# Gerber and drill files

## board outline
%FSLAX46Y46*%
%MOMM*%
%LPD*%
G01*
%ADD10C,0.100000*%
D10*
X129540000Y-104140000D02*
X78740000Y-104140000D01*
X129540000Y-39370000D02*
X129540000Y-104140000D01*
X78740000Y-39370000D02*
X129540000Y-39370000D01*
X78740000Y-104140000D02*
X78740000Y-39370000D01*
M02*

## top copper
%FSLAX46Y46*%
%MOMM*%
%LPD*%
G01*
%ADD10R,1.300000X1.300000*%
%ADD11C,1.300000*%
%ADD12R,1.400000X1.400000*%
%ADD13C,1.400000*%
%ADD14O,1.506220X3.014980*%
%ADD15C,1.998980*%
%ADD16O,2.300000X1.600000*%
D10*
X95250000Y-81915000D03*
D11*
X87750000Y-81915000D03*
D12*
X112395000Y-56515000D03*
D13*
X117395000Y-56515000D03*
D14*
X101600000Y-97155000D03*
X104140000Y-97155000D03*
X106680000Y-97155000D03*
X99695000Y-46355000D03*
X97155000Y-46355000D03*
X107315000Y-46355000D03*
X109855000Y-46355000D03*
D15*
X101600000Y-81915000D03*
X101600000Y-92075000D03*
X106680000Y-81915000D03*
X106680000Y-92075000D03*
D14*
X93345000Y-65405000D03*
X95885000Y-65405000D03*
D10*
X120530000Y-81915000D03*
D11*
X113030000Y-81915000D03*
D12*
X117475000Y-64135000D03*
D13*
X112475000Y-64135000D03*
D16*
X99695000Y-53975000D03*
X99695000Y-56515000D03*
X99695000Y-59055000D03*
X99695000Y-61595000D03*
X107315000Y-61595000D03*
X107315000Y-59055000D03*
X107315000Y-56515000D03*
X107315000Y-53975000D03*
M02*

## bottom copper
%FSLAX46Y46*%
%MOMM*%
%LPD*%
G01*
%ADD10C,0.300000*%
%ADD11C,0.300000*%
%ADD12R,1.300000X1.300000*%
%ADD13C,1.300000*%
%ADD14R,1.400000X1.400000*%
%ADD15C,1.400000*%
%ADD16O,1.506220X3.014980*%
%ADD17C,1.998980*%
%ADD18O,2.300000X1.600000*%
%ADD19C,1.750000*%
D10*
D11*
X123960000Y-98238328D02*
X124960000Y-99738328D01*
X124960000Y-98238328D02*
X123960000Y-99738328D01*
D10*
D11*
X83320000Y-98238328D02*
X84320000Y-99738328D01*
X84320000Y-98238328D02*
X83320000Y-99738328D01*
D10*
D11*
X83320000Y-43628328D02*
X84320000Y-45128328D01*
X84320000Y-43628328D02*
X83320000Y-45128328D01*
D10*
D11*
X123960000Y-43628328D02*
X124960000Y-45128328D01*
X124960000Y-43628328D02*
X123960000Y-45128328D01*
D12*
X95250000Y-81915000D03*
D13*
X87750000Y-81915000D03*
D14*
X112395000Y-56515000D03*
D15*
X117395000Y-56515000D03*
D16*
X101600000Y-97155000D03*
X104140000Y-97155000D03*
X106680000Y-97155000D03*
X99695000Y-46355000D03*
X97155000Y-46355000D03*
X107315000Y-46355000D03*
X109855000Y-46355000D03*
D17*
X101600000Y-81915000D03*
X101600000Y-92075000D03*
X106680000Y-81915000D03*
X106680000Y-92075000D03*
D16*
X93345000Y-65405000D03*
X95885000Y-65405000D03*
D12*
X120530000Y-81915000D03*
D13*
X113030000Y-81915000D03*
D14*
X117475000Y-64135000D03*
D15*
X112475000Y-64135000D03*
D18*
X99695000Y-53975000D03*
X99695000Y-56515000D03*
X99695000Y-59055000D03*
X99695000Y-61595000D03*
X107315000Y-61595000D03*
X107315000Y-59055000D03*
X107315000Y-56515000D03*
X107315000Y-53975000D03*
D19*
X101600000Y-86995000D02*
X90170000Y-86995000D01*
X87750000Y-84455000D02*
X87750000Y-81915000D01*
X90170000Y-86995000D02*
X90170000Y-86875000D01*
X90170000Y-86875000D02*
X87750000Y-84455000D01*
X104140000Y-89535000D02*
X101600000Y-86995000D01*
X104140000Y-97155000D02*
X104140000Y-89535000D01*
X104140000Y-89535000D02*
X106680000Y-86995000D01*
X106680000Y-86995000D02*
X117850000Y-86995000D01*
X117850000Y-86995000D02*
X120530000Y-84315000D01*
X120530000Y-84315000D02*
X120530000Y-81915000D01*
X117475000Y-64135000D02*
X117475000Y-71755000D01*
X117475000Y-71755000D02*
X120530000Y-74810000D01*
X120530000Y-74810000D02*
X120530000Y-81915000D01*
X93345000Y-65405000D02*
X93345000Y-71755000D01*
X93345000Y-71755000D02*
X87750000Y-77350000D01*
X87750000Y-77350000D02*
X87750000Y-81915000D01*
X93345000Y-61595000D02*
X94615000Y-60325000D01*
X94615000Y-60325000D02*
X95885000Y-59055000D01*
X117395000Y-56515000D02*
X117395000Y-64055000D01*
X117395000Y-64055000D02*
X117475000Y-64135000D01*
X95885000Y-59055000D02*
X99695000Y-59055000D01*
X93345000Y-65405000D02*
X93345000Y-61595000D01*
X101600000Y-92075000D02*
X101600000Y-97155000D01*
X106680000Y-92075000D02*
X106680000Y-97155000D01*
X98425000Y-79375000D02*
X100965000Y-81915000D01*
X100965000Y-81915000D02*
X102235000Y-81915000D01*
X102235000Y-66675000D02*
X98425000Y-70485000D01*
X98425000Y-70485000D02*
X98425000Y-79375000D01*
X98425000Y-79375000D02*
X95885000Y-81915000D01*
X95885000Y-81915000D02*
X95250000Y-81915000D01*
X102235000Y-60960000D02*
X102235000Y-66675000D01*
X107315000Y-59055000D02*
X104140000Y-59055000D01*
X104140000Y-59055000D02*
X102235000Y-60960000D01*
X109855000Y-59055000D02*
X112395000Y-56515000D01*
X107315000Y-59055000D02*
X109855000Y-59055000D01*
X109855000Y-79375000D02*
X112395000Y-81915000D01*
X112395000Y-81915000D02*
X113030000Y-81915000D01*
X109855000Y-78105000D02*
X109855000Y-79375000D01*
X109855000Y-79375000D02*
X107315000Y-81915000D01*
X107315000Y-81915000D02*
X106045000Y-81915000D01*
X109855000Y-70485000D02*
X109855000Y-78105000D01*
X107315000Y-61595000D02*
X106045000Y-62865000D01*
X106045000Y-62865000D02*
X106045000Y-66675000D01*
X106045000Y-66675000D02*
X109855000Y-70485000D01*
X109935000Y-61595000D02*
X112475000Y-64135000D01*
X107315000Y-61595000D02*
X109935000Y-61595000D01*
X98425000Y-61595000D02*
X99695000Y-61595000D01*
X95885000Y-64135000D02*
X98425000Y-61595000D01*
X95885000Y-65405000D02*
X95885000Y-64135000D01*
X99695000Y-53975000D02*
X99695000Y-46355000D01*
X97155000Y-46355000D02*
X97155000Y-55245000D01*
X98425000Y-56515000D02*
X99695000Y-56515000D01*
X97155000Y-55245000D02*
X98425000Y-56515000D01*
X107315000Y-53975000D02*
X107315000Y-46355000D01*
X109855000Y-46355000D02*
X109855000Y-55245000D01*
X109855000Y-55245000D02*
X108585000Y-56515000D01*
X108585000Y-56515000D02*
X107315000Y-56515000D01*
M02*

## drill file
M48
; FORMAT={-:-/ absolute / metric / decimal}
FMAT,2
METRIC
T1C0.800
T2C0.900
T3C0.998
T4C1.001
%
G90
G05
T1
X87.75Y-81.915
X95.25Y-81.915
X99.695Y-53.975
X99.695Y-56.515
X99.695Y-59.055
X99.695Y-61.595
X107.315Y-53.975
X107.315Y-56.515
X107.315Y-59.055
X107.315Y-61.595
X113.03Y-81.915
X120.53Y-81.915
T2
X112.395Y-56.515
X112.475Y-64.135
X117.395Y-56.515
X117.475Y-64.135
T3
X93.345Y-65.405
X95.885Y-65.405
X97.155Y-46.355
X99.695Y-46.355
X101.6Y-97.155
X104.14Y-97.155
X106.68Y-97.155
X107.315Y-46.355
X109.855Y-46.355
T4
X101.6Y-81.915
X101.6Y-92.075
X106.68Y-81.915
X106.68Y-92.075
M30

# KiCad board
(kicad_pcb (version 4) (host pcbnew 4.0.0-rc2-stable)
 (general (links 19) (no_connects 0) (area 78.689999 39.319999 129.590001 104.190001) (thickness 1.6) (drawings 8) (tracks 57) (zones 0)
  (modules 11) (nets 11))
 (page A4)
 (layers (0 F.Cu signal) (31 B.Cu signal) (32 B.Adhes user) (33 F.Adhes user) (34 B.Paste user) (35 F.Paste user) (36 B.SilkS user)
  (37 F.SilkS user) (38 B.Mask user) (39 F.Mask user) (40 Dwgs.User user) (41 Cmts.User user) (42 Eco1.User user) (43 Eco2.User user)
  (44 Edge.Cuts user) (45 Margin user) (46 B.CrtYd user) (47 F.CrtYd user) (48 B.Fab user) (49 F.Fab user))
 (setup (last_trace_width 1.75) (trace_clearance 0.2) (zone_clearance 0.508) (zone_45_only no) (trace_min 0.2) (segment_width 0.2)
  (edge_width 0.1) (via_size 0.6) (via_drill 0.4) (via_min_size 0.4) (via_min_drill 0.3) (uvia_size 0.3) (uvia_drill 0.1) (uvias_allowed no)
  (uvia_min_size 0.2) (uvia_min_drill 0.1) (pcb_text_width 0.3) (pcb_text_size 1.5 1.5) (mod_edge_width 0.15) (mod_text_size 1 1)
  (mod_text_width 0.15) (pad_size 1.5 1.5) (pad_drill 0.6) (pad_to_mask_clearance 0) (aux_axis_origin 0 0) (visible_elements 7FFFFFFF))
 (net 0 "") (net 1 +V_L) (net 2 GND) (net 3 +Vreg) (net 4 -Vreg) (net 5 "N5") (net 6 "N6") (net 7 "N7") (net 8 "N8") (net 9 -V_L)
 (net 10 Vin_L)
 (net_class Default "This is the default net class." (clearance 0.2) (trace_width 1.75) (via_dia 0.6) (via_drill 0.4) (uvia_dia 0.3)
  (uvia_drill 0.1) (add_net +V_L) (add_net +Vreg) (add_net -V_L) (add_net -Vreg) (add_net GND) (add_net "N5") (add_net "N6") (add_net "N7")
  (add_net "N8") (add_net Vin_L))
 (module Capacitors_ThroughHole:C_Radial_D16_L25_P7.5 (layer F.Cu) (at 95.25 81.915 180)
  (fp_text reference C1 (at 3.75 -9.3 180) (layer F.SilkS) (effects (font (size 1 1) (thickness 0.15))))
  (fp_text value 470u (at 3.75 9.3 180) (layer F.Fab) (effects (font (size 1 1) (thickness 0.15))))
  (pad 1 thru_hole rect (at 0 0 180) (size 1.3 1.3) (drill 0.8) (layers *.Cu *.Mask F.SilkS) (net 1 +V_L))
  (pad 2 thru_hole circle (at 7.5 0 180) (size 1.3 1.3) (drill 0.8) (layers *.Cu *.Mask F.SilkS) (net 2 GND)))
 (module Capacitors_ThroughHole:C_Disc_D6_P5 (layer F.Cu) (at 112.395 56.515)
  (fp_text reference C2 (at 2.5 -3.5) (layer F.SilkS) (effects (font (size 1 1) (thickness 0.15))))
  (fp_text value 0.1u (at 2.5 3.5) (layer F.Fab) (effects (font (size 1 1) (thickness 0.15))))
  (pad 1 thru_hole rect (at 0 0) (size 1.4 1.4) (drill 0.9) (layers *.Cu *.Mask F.SilkS) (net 1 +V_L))
  (pad 2 thru_hole circle (at 5 0) (size 1.4 1.4) (drill 0.9) (layers *.Cu *.Mask F.SilkS) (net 2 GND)))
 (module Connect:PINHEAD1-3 (layer F.Cu) (at 104.14 97.155)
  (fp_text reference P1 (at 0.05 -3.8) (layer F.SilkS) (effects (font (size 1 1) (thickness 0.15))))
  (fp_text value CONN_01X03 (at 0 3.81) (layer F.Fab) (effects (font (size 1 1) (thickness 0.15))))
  (pad 1 thru_hole oval (at -2.54 0) (size 1.50622 3.01498) (drill 0.99822) (layers *.Cu *.Mask) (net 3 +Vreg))
  (pad 2 thru_hole oval (at 0 0) (size 1.50622 3.01498) (drill 0.99822) (layers *.Cu *.Mask) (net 2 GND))
  (pad 3 thru_hole oval (at 2.54 0) (size 1.50622 3.01498) (drill 0.99822) (layers *.Cu *.Mask) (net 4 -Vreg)))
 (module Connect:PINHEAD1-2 (layer F.Cu) (at 98.425 46.355 180)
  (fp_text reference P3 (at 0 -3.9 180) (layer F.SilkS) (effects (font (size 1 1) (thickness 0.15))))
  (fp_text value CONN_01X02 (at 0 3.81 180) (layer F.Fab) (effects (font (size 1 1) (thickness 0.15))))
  (pad 1 thru_hole oval (at -1.27 0 180) (size 1.50622 3.01498) (drill 0.99822) (layers *.Cu *.Mask) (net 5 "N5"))
  (pad 2 thru_hole oval (at 1.27 0 180) (size 1.50622 3.01498) (drill 0.99822) (layers *.Cu *.Mask) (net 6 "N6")))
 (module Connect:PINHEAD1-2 (layer F.Cu) (at 108.585 46.355)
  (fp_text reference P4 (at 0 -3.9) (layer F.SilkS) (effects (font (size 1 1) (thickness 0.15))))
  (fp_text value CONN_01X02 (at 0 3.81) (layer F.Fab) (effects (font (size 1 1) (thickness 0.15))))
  (pad 1 thru_hole oval (at -1.27 0) (size 1.50622 3.01498) (drill 0.99822) (layers *.Cu *.Mask) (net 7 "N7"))
  (pad 2 thru_hole oval (at 1.27 0) (size 1.50622 3.01498) (drill 0.99822) (layers *.Cu *.Mask) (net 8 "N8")))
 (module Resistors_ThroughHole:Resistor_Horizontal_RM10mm (layer F.Cu) (at 101.6 86.995 270)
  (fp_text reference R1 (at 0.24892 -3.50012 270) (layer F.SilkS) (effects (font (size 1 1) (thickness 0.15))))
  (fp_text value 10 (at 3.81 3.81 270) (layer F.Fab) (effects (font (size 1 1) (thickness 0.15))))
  (pad 1 thru_hole circle (at -5.08 0 270) (size 1.99898 1.99898) (drill 1.00076) (layers *.Cu *.SilkS *.Mask) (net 1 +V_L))
  (pad 2 thru_hole circle (at 5.08 0 270) (size 1.99898 1.99898) (drill 1.00076) (layers *.Cu *.SilkS *.Mask) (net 3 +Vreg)))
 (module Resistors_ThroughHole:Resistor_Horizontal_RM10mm (layer F.Cu) (at 106.68 86.995 270)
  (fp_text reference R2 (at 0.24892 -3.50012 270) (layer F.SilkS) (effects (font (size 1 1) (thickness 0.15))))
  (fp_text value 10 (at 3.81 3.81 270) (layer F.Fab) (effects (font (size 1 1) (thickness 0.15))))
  (pad 1 thru_hole circle (at -5.08 0 270) (size 1.99898 1.99898) (drill 1.00076) (layers *.Cu *.SilkS *.Mask) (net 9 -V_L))
  (pad 2 thru_hole circle (at 5.08 0 270) (size 1.99898 1.99898) (drill 1.00076) (layers *.Cu *.SilkS *.Mask) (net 4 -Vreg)))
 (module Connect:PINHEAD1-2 (layer F.Cu) (at 94.615 65.405)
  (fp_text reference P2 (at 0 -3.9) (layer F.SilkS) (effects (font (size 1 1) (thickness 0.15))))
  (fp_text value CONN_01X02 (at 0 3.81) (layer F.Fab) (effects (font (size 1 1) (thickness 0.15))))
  (pad 1 thru_hole oval (at -1.27 0) (size 1.50622 3.01498) (drill 0.99822) (layers *.Cu *.Mask) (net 2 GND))
  (pad 2 thru_hole oval (at 1.27 0) (size 1.50622 3.01498) (drill 0.99822) (layers *.Cu *.Mask) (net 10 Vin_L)))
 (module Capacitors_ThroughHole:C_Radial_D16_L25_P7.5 (layer F.Cu) (at 120.53 81.915 180)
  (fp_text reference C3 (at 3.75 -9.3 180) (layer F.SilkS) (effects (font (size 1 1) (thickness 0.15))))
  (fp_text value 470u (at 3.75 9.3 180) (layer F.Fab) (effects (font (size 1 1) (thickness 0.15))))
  (pad 1 thru_hole rect (at 0 0 180) (size 1.3 1.3) (drill 0.8) (layers *.Cu *.Mask F.SilkS) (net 2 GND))
  (pad 2 thru_hole circle (at 7.5 0 180) (size 1.3 1.3) (drill 0.8) (layers *.Cu *.Mask F.SilkS) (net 9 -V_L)))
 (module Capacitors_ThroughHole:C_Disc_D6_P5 (layer F.Cu) (at 117.475 64.135 180)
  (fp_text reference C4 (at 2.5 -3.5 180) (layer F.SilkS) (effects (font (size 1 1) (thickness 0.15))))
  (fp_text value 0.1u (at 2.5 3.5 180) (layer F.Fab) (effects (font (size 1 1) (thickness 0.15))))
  (pad 1 thru_hole rect (at 0 0 180) (size 1.4 1.4) (drill 0.9) (layers *.Cu *.Mask F.SilkS) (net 2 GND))
  (pad 2 thru_hole circle (at 5 0 180) (size 1.4 1.4) (drill 0.9) (layers *.Cu *.Mask F.SilkS) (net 9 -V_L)))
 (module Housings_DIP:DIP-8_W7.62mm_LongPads (layer F.Cu) (at 99.695 53.975)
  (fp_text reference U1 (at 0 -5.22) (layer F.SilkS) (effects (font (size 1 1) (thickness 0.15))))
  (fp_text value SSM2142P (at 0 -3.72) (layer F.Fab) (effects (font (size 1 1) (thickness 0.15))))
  (pad 1 thru_hole oval (at 0 0) (size 2.3 1.6) (drill 0.8) (layers *.Cu *.Mask F.SilkS) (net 5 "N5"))
  (pad 2 thru_hole oval (at 0 2.54) (size 2.3 1.6) (drill 0.8) (layers *.Cu *.Mask F.SilkS) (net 6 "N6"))
  (pad 3 thru_hole oval (at 0 5.08) (size 2.3 1.6) (drill 0.8) (layers *.Cu *.Mask F.SilkS) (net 2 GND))
  (pad 4 thru_hole oval (at 0 7.62) (size 2.3 1.6) (drill 0.8) (layers *.Cu *.Mask F.SilkS) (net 10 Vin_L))
  (pad 5 thru_hole oval (at 7.62 7.62) (size 2.3 1.6) (drill 0.8) (layers *.Cu *.Mask F.SilkS) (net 9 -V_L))
  (pad 6 thru_hole oval (at 7.62 5.08) (size 2.3 1.6) (drill 0.8) (layers *.Cu *.Mask F.SilkS) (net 1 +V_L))
  (pad 7 thru_hole oval (at 7.62 2.54) (size 2.3 1.6) (drill 0.8) (layers *.Cu *.Mask F.SilkS) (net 8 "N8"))
  (pad 8 thru_hole oval (at 7.62 0) (size 2.3 1.6) (drill 0.8) (layers *.Cu *.Mask F.SilkS) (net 7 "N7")))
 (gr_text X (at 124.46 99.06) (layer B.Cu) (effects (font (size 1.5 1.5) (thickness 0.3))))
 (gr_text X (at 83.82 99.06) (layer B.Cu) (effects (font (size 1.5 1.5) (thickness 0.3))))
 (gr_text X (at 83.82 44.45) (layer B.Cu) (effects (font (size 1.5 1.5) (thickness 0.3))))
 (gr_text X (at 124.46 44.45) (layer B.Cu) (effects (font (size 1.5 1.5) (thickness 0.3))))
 (gr_line (start 129.54 104.14) (end 78.74 104.14) (angle 90) (layer Edge.Cuts) (width 0.1))
 (gr_line (start 129.54 39.37) (end 129.54 104.14) (angle 90) (layer Edge.Cuts) (width 0.1))
 (gr_line (start 78.74 39.37) (end 129.54 39.37) (angle 90) (layer Edge.Cuts) (width 0.1))
 (gr_line (start 78.74 104.14) (end 78.74 39.37) (angle 90) (layer Edge.Cuts) (width 0.1))
 (segment (start 101.6 86.995) (end 90.17 86.995) (width 1.75) (layer B.Cu) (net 2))
 (segment (start 87.75 84.455) (end 87.75 81.915) (width 1.75) (layer B.Cu) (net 2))
 (segment (start 90.17 86.995) (end 90.17 86.875) (width 1.75) (layer B.Cu) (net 2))
 (segment (start 90.17 86.875) (end 87.75 84.455) (width 1.75) (layer B.Cu) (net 2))
 (segment (start 104.14 89.535) (end 101.6 86.995) (width 1.75) (layer B.Cu) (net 2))
 (segment (start 104.14 97.155) (end 104.14 89.535) (width 1.75) (layer B.Cu) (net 2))
 (segment (start 104.14 89.535) (end 106.68 86.995) (width 1.75) (layer B.Cu) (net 2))
 (segment (start 106.68 86.995) (end 117.85 86.995) (width 1.75) (layer B.Cu) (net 2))
 (segment (start 117.85 86.995) (end 120.53 84.315) (width 1.75) (layer B.Cu) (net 2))
 (segment (start 120.53 84.315) (end 120.53 81.915) (width 1.75) (layer B.Cu) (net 2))
 (segment (start 117.475 64.135) (end 117.475 71.755) (width 1.75) (layer B.Cu) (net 2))
 (segment (start 117.475 71.755) (end 120.53 74.81) (width 1.75) (layer B.Cu) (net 2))
 (segment (start 120.53 74.81) (end 120.53 81.915) (width 1.75) (layer B.Cu) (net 2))
 (segment (start 93.345 65.405) (end 93.345 71.755) (width 1.75) (layer B.Cu) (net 2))
 (segment (start 93.345 71.755) (end 87.75 77.35) (width 1.75) (layer B.Cu) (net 2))
 (segment (start 87.75 77.35) (end 87.75 81.915) (width 1.75) (layer B.Cu) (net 2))
 (segment (start 93.345 61.595) (end 94.615 60.325) (width 1.75) (layer B.Cu) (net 2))
 (segment (start 94.615 60.325) (end 95.885 59.055) (width 1.75) (layer B.Cu) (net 2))
 (segment (start 117.395 56.515) (end 117.395 64.055) (width 1.75) (layer B.Cu) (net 2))
 (segment (start 117.395 64.055) (end 117.475 64.135) (width 1.75) (layer B.Cu) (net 2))
 (segment (start 95.885 59.055) (end 99.695 59.055) (width 1.75) (layer B.Cu) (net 2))
 (segment (start 93.345 65.405) (end 93.345 61.595) (width 1.75) (layer B.Cu) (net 2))
 (segment (start 101.6 92.075) (end 101.6 97.155) (width 1.75) (layer B.Cu) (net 3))
 (segment (start 106.68 92.075) (end 106.68 97.155) (width 1.75) (layer B.Cu) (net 4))
 (segment (start 98.425 79.375) (end 100.965 81.915) (width 1.75) (layer B.Cu) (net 1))
 (segment (start 100.965 81.915) (end 102.235 81.915) (width 1.75) (layer B.Cu) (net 1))
 (segment (start 102.235 66.675) (end 98.425 70.485) (width 1.75) (layer B.Cu) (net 1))
 (segment (start 98.425 70.485) (end 98.425 79.375) (width 1.75) (layer B.Cu) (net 1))
 (segment (start 98.425 79.375) (end 95.885 81.915) (width 1.75) (layer B.Cu) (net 1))
 (segment (start 95.885 81.915) (end 95.25 81.915) (width 1.75) (layer B.Cu) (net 1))
 (segment (start 102.235 60.96) (end 102.235 66.675) (width 1.75) (layer B.Cu) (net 1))
 (segment (start 107.315 59.055) (end 104.14 59.055) (width 1.75) (layer B.Cu) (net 1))
 (segment (start 104.14 59.055) (end 102.235 60.96) (width 1.75) (layer B.Cu) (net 1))
 (segment (start 109.855 59.055) (end 112.395 56.515) (width 1.75) (layer B.Cu) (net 1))
 (segment (start 107.315 59.055) (end 109.855 59.055) (width 1.75) (layer B.Cu) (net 1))
 (segment (start 109.855 79.375) (end 112.395 81.915) (width 1.75) (layer B.Cu) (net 9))
 (segment (start 112.395 81.915) (end 113.03 81.915) (width 1.75) (layer B.Cu) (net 9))
 (segment (start 109.855 78.105) (end 109.855 79.375) (width 1.75) (layer B.Cu) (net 9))
 (segment (start 109.855 79.375) (end 107.315 81.915) (width 1.75) (layer B.Cu) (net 9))
 (segment (start 107.315 81.915) (end 106.045 81.915) (width 1.75) (layer B.Cu) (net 9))
 (segment (start 109.855 70.485) (end 109.855 78.105) (width 1.75) (layer B.Cu) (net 9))
 (segment (start 107.315 61.595) (end 106.045 62.865) (width 1.75) (layer B.Cu) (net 9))
 (segment (start 106.045 62.865) (end 106.045 66.675) (width 1.75) (layer B.Cu) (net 9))
 (segment (start 106.045 66.675) (end 109.855 70.485) (width 1.75) (layer B.Cu) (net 9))
 (segment (start 109.935 61.595) (end 112.475 64.135) (width 1.75) (layer B.Cu) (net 9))
 (segment (start 107.315 61.595) (end 109.935 61.595) (width 1.75) (layer B.Cu) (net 9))
 (segment (start 98.425 61.595) (end 99.695 61.595) (width 1.75) (layer B.Cu) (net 10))
 (segment (start 95.885 64.135) (end 98.425 61.595) (width 1.75) (layer B.Cu) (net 10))
 (segment (start 95.885 65.405) (end 95.885 64.135) (width 1.75) (layer B.Cu) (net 10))
 (segment (start 99.695 53.975) (end 99.695 46.355) (width 1.75) (layer B.Cu) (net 5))
 (segment (start 97.155 46.355) (end 97.155 55.245) (width 1.75) (layer B.Cu) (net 6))
 (segment (start 98.425 56.515) (end 99.695 56.515) (width 1.75) (layer B.Cu) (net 6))
 (segment (start 97.155 55.245) (end 98.425 56.515) (width 1.75) (layer B.Cu) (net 6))
 (segment (start 107.315 53.975) (end 107.315 46.355) (width 1.75) (layer B.Cu) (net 7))
 (segment (start 109.855 46.355) (end 109.855 55.245) (width 1.75) (layer B.Cu) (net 8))
 (segment (start 109.855 55.245) (end 108.585 56.515) (width 1.75) (layer B.Cu) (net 8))
 (segment (start 108.585 56.515) (end 107.315 56.515) (width 1.75) (layer B.Cu) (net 8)))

